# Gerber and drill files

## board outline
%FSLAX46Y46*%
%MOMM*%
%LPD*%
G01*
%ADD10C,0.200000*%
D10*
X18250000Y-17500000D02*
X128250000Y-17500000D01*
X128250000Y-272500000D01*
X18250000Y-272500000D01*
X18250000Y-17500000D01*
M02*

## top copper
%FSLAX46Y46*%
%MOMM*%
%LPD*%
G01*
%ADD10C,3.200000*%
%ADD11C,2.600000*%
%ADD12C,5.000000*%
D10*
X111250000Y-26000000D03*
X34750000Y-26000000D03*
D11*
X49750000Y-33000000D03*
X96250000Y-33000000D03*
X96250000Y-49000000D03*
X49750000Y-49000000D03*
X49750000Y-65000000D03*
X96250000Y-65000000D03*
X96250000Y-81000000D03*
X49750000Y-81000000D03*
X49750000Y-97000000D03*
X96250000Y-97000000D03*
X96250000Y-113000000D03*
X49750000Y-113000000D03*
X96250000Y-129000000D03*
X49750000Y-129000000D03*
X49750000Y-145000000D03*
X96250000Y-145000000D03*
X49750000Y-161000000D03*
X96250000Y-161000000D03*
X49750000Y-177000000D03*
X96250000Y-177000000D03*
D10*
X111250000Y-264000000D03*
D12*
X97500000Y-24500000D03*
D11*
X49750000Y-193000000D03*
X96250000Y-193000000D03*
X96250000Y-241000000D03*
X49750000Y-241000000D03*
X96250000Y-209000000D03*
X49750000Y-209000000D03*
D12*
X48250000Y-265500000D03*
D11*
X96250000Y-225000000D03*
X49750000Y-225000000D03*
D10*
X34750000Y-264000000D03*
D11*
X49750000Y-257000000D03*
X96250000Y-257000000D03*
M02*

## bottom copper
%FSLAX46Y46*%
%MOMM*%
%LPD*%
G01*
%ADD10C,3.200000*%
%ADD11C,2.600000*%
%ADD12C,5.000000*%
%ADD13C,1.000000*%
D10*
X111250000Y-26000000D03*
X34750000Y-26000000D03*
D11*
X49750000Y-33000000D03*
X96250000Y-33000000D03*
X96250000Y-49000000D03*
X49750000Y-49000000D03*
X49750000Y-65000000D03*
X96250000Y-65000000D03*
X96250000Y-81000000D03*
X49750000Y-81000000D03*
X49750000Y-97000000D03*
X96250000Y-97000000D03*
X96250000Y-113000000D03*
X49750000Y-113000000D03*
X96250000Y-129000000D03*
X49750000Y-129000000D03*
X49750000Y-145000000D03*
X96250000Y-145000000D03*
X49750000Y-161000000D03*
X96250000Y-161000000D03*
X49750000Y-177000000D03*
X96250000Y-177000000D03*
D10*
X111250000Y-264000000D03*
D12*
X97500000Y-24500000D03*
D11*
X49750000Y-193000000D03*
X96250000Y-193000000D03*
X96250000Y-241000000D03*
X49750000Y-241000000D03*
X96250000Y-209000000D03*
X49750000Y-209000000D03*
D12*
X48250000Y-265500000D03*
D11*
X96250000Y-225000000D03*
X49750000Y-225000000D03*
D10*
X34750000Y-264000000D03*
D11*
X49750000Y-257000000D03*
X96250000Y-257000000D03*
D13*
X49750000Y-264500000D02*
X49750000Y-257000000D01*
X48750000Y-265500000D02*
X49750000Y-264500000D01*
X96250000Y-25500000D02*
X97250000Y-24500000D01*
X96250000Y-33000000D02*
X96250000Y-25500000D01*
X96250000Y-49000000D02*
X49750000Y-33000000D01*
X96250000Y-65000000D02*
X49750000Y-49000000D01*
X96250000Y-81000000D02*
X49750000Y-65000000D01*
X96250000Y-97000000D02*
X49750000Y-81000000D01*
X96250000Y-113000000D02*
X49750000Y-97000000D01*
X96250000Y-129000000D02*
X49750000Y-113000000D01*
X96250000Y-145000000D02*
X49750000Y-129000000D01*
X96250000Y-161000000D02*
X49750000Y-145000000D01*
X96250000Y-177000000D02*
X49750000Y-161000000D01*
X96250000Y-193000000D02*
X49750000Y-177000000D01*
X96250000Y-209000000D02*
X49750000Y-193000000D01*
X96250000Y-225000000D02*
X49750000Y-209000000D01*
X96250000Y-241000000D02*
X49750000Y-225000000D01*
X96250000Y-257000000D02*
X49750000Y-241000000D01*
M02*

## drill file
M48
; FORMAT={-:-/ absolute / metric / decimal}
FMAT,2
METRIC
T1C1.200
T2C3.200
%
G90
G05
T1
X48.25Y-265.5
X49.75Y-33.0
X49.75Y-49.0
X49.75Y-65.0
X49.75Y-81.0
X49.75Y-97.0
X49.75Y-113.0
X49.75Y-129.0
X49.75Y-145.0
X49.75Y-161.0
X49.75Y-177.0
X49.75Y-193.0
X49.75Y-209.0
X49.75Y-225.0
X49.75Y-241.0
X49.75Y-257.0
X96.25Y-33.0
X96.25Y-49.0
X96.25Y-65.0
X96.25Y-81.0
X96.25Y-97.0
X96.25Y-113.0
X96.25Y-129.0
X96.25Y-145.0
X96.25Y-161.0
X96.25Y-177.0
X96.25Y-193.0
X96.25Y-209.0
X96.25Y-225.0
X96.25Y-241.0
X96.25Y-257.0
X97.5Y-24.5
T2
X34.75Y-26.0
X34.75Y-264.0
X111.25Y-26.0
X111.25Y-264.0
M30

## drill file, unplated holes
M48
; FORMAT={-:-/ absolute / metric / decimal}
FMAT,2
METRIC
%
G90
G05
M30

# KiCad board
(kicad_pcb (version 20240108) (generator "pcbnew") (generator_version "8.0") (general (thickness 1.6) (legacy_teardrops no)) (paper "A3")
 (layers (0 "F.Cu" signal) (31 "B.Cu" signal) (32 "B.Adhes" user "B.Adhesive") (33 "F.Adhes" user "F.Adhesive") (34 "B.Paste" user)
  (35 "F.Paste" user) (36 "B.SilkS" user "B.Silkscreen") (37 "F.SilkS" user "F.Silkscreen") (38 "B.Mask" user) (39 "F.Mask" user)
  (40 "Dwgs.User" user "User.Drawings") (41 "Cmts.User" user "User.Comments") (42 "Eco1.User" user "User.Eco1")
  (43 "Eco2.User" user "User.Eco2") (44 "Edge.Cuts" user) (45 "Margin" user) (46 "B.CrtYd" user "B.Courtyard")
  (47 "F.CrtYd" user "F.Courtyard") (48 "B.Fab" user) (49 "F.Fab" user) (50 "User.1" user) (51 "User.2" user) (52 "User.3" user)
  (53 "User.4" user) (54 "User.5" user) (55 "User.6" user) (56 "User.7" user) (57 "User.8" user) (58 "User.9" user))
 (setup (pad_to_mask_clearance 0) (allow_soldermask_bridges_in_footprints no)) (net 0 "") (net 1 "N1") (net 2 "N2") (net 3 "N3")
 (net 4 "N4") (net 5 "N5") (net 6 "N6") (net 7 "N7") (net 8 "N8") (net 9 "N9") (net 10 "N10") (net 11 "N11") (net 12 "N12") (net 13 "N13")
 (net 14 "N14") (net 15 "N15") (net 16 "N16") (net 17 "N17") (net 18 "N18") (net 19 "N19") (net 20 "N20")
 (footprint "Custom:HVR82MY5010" (layer "F.Cu") (at 73 177 180)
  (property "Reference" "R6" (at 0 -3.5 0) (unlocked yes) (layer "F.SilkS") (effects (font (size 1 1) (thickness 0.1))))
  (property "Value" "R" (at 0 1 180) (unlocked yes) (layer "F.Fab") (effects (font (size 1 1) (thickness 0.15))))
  (pad "1" thru_hole circle (at -23.25 0 180) (size 2.6 2.6) (drill 1.2) (layers "*.Cu" "*.Mask") (remove_unused_layers no) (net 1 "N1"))
  (pad "2" thru_hole circle (at 23.25 0 180) (size 2.6 2.6) (drill 1.2) (layers "*.Cu" "*.Mask") (remove_unused_layers no) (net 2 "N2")))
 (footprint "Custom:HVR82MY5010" (layer "F.Cu") (at 73 65 180)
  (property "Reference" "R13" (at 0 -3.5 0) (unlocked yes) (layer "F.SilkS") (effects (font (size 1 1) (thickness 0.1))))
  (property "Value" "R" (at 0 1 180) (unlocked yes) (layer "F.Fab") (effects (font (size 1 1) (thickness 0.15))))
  (pad "1" thru_hole circle (at -23.25 0 180) (size 2.6 2.6) (drill 1.2) (layers "*.Cu" "*.Mask") (remove_unused_layers no) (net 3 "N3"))
  (pad "2" thru_hole circle (at 23.25 0 180) (size 2.6 2.6) (drill 1.2) (layers "*.Cu" "*.Mask") (remove_unused_layers no) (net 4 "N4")))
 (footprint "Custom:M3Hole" (layer "F.Cu") (at 111.25 264)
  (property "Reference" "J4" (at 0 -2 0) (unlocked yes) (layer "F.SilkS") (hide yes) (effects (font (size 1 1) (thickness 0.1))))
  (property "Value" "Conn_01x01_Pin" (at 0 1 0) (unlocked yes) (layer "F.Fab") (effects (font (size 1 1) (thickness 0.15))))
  (pad "1" thru_hole circle (at 0 0) (size 3.2 3.2) (drill 3.2) (layers "*.Cu" "*.Mask") (remove_unused_layers no) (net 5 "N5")))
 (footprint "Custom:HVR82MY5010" (layer "F.Cu") (at 73 33 180)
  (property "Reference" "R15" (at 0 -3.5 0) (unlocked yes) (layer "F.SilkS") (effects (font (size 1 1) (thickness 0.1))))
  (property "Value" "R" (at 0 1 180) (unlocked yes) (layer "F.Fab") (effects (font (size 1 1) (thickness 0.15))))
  (pad "1" thru_hole circle (at -23.25 0 180) (size 2.6 2.6) (drill 1.2) (layers "*.Cu" "*.Mask") (remove_unused_layers no) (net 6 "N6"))
  (pad "2" thru_hole circle (at 23.25 0 180) (size 2.6 2.6) (drill 1.2) (layers "*.Cu" "*.Mask") (remove_unused_layers no) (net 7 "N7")))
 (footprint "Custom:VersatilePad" (layer "F.Cu") (at 97.5 -101.5)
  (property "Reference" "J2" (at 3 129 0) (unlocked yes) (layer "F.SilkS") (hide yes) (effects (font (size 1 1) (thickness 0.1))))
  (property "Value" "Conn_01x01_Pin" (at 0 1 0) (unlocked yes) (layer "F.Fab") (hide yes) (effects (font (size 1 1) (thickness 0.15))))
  (pad "1" thru_hole circle (at 0 126) (size 5 5) (drill 1.2) (layers "*.Cu" "*.Mask") (remove_unused_layers no) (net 6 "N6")))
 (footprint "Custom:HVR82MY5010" (layer "F.Cu") (at 73 49)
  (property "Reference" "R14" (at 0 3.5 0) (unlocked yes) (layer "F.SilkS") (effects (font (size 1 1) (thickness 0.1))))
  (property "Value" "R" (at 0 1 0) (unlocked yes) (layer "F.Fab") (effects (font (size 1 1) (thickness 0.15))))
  (pad "1" thru_hole circle (at -23.25 0) (size 2.6 2.6) (drill 1.2) (layers "*.Cu" "*.Mask") (remove_unused_layers no) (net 3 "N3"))
  (pad "2" thru_hole circle (at 23.25 0) (size 2.6 2.6) (drill 1.2) (layers "*.Cu" "*.Mask") (remove_unused_layers no) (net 7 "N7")))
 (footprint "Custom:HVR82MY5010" (layer "F.Cu") (at 73 193 180)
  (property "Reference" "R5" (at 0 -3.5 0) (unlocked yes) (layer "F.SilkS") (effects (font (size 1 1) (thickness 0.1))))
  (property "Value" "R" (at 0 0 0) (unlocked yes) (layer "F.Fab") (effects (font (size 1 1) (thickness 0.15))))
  (pad "1" thru_hole circle (at -23.25 0 180) (size 2.6 2.6) (drill 1.2) (layers "*.Cu" "*.Mask") (remove_unused_layers no) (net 2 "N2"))
  (pad "2" thru_hole circle (at 23.25 0 180) (size 2.6 2.6) (drill 1.2) (layers "*.Cu" "*.Mask") (remove_unused_layers no) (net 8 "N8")))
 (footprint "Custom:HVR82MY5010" (layer "F.Cu") (at 73 241)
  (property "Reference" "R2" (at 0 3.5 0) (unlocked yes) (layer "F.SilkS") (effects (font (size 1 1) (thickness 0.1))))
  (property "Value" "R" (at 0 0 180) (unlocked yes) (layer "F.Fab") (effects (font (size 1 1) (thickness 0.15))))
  (pad "1" thru_hole circle (at -23.25 0) (size 2.6 2.6) (drill 1.2) (layers "*.Cu" "*.Mask") (remove_unused_layers no) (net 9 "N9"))
  (pad "2" thru_hole circle (at 23.25 0) (size 2.6 2.6) (drill 1.2) (layers "*.Cu" "*.Mask") (remove_unused_layers no) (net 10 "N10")))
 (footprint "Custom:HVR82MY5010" (layer "F.Cu") (at 73 209)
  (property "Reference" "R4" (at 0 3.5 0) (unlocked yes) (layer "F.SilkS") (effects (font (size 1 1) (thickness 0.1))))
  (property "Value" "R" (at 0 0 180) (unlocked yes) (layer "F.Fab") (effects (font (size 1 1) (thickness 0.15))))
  (pad "1" thru_hole circle (at -23.25 0) (size 2.6 2.6) (drill 1.2) (layers "*.Cu" "*.Mask") (remove_unused_layers no) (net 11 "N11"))
  (pad "2" thru_hole circle (at 23.25 0) (size 2.6 2.6) (drill 1.2) (layers "*.Cu" "*.Mask") (remove_unused_layers no) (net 8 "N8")))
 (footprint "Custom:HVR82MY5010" (layer "F.Cu") (at 73 161)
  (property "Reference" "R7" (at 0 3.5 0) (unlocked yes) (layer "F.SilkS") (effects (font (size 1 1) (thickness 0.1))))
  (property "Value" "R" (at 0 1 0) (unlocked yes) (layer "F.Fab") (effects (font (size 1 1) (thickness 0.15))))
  (pad "1" thru_hole circle (at -23.25 0) (size 2.6 2.6) (drill 1.2) (layers "*.Cu" "*.Mask") (remove_unused_layers no) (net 1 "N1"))
  (pad "2" thru_hole circle (at 23.25 0) (size 2.6 2.6) (drill 1.2) (layers "*.Cu" "*.Mask") (remove_unused_layers no) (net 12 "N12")))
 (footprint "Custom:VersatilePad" (layer "F.Cu") (at 48.25 265.5)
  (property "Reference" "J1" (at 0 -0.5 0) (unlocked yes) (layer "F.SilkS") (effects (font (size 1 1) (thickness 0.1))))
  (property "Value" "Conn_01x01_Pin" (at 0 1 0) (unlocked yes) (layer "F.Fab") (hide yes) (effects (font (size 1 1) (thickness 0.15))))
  (pad "1" thru_hole circle (at 0 0) (size 5 5) (drill 1.2) (layers "*.Cu" "*.Mask") (remove_unused_layers no) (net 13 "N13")))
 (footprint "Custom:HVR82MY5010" (layer "F.Cu") (at 73 225 180)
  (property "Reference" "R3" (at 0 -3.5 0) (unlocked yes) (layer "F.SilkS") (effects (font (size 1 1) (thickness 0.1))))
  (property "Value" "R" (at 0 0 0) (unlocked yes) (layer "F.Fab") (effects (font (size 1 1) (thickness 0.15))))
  (pad "1" thru_hole circle (at -23.25 0 180) (size 2.6 2.6) (drill 1.2) (layers "*.Cu" "*.Mask") (remove_unused_layers no) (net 11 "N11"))
  (pad "2" thru_hole circle (at 23.25 0 180) (size 2.6 2.6) (drill 1.2) (layers "*.Cu" "*.Mask") (remove_unused_layers no) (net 10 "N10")))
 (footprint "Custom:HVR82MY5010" (layer "F.Cu") (at 73 81)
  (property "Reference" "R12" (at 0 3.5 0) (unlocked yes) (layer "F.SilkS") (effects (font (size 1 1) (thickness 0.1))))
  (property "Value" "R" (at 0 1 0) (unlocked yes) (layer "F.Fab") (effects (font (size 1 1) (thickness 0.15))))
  (pad "1" thru_hole circle (at -23.25 0) (size 2.6 2.6) (drill 1.2) (layers "*.Cu" "*.Mask") (remove_unused_layers no) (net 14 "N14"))
  (pad "2" thru_hole circle (at 23.25 0) (size 2.6 2.6) (drill 1.2) (layers "*.Cu" "*.Mask") (remove_unused_layers no) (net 4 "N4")))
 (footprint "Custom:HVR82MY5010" (layer "F.Cu") (at 73 113 180)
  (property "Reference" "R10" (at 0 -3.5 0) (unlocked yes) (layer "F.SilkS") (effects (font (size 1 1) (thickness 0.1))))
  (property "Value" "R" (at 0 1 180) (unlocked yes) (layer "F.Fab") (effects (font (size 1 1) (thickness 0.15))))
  (pad "1" thru_hole circle (at -23.25 0 180) (size 2.6 2.6) (drill 1.2) (layers "*.Cu" "*.Mask") (remove_unused_layers no) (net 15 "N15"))
  (pad "2" thru_hole circle (at 23.25 0 180) (size 2.6 2.6) (drill 1.2) (layers "*.Cu" "*.Mask") (remove_unused_layers no) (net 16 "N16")))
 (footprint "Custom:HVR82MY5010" (layer "F.Cu") (at 73 97 180)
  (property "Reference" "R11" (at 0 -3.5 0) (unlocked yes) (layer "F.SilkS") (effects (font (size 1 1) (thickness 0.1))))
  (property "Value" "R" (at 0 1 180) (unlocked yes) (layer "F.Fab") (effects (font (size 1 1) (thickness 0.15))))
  (pad "1" thru_hole circle (at -23.25 0 180) (size 2.6 2.6) (drill 1.2) (layers "*.Cu" "*.Mask") (remove_unused_layers no) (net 14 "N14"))
  (pad "2" thru_hole circle (at 23.25 0 180) (size 2.6 2.6) (drill 1.2) (layers "*.Cu" "*.Mask") (remove_unused_layers no) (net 15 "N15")))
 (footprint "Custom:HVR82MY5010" (layer "F.Cu") (at 73 129)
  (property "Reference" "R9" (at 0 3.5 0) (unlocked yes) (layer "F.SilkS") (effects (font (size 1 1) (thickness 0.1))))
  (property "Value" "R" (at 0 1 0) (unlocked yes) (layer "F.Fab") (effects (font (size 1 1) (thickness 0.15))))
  (pad "1" thru_hole circle (at -23.25 0) (size 2.6 2.6) (drill 1.2) (layers "*.Cu" "*.Mask") (remove_unused_layers no) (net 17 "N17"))
  (pad "2" thru_hole circle (at 23.25 0) (size 2.6 2.6) (drill 1.2) (layers "*.Cu" "*.Mask") (remove_unused_layers no) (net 16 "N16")))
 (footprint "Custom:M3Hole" (layer "F.Cu") (at 34.75 264)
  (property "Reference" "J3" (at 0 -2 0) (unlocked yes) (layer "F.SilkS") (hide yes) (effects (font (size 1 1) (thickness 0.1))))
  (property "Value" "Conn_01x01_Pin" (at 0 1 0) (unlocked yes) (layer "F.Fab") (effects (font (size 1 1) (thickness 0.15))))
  (pad "1" thru_hole circle (at 0 0) (size 3.2 3.2) (drill 3.2) (layers "*.Cu" "*.Mask") (remove_unused_layers no) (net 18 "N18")))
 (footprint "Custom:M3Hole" (layer "F.Cu") (at 34.75 26)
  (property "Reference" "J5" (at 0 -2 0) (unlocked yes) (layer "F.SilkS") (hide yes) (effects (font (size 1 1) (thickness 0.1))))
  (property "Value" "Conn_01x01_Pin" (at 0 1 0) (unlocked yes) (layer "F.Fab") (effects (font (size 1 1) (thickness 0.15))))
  (pad "1" thru_hole circle (at 0 0) (size 3.2 3.2) (drill 3.2) (layers "*.Cu" "*.Mask") (remove_unused_layers no) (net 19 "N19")))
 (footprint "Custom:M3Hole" (layer "F.Cu") (at 111.25 26)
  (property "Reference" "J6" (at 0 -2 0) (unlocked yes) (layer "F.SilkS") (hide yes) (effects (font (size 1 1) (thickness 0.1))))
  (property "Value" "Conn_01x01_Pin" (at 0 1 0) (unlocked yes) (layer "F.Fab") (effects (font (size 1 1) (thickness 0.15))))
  (pad "1" thru_hole circle (at 0 0) (size 3.2 3.2) (drill 3.2) (layers "*.Cu" "*.Mask") (remove_unused_layers no) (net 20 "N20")))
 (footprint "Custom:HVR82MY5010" (layer "F.Cu") (at 73 257 180)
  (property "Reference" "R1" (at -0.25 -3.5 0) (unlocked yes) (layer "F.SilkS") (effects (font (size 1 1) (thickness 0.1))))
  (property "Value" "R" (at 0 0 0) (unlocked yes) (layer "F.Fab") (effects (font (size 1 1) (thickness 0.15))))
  (pad "1" thru_hole circle (at -23.25 0 180) (size 2.6 2.6) (drill 1.2) (layers "*.Cu" "*.Mask") (remove_unused_layers no) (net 9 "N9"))
  (pad "2" thru_hole circle (at 23.25 0 180) (size 2.6 2.6) (drill 1.2) (layers "*.Cu" "*.Mask") (remove_unused_layers no) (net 13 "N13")))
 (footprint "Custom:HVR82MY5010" (layer "F.Cu") (at 73 145 180)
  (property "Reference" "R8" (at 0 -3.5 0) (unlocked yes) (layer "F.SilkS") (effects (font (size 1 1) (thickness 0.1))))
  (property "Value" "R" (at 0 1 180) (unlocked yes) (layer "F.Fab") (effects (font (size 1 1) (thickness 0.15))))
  (pad "1" thru_hole circle (at -23.25 0 180) (size 2.6 2.6) (drill 1.2) (layers "*.Cu" "*.Mask") (remove_unused_layers no) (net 17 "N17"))
  (pad "2" thru_hole circle (at 23.25 0 180) (size 2.6 2.6) (drill 1.2) (layers "*.Cu" "*.Mask") (remove_unused_layers no) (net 12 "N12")))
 (gr_rect (start 18.25 17.5) (end 128.25 272.5) (stroke (width 0.2) (type default)) (fill none) (layer "Edge.Cuts"))
 (segment (start 49.75 264.5) (end 49.75 257) (width 1) (layer "B.Cu") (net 13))
 (segment (start 48.75 265.5) (end 49.75 264.5) (width 1) (layer "B.Cu") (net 13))
 (segment (start 96.25 25.5) (end 97.25 24.5) (width 1) (layer "B.Cu") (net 6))
 (segment (start 96.25 33) (end 96.25 25.5) (width 1) (layer "B.Cu") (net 6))
 (segment (start 96.25 257) (end 49.75 241) (width 1) (layer "B.Cu") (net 9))
 (segment (start 96.25 241) (end 49.75 225) (width 1) (layer "B.Cu") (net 10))
 (segment (start 96.25 225) (end 49.75 209) (width 1) (layer "B.Cu") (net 11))
 (segment (start 96.25 209) (end 49.75 193) (width 1) (layer "B.Cu") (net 8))
 (segment (start 96.25 193) (end 49.75 177) (width 1) (layer "B.Cu") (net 2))
 (segment (start 96.25 177) (end 49.75 161) (width 1) (layer "B.Cu") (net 1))
 (segment (start 96.25 161) (end 49.75 145) (width 1) (layer "B.Cu") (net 12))
 (segment (start 96.25 145) (end 49.75 129) (width 1) (layer "B.Cu") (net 17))
 (segment (start 96.25 129) (end 49.75 113) (width 1) (layer "B.Cu") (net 16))
 (segment (start 96.25 113) (end 49.75 97) (width 1) (layer "B.Cu") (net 15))
 (segment (start 96.25 97) (end 49.75 81) (width 1) (layer "B.Cu") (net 14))
 (segment (start 96.25 81) (end 49.75 65) (width 1) (layer "B.Cu") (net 4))
 (segment (start 96.25 65) (end 49.75 49) (width 1) (layer "B.Cu") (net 3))
 (segment (start 96.25 49) (end 49.75 33) (width 1) (layer "B.Cu") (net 7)))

